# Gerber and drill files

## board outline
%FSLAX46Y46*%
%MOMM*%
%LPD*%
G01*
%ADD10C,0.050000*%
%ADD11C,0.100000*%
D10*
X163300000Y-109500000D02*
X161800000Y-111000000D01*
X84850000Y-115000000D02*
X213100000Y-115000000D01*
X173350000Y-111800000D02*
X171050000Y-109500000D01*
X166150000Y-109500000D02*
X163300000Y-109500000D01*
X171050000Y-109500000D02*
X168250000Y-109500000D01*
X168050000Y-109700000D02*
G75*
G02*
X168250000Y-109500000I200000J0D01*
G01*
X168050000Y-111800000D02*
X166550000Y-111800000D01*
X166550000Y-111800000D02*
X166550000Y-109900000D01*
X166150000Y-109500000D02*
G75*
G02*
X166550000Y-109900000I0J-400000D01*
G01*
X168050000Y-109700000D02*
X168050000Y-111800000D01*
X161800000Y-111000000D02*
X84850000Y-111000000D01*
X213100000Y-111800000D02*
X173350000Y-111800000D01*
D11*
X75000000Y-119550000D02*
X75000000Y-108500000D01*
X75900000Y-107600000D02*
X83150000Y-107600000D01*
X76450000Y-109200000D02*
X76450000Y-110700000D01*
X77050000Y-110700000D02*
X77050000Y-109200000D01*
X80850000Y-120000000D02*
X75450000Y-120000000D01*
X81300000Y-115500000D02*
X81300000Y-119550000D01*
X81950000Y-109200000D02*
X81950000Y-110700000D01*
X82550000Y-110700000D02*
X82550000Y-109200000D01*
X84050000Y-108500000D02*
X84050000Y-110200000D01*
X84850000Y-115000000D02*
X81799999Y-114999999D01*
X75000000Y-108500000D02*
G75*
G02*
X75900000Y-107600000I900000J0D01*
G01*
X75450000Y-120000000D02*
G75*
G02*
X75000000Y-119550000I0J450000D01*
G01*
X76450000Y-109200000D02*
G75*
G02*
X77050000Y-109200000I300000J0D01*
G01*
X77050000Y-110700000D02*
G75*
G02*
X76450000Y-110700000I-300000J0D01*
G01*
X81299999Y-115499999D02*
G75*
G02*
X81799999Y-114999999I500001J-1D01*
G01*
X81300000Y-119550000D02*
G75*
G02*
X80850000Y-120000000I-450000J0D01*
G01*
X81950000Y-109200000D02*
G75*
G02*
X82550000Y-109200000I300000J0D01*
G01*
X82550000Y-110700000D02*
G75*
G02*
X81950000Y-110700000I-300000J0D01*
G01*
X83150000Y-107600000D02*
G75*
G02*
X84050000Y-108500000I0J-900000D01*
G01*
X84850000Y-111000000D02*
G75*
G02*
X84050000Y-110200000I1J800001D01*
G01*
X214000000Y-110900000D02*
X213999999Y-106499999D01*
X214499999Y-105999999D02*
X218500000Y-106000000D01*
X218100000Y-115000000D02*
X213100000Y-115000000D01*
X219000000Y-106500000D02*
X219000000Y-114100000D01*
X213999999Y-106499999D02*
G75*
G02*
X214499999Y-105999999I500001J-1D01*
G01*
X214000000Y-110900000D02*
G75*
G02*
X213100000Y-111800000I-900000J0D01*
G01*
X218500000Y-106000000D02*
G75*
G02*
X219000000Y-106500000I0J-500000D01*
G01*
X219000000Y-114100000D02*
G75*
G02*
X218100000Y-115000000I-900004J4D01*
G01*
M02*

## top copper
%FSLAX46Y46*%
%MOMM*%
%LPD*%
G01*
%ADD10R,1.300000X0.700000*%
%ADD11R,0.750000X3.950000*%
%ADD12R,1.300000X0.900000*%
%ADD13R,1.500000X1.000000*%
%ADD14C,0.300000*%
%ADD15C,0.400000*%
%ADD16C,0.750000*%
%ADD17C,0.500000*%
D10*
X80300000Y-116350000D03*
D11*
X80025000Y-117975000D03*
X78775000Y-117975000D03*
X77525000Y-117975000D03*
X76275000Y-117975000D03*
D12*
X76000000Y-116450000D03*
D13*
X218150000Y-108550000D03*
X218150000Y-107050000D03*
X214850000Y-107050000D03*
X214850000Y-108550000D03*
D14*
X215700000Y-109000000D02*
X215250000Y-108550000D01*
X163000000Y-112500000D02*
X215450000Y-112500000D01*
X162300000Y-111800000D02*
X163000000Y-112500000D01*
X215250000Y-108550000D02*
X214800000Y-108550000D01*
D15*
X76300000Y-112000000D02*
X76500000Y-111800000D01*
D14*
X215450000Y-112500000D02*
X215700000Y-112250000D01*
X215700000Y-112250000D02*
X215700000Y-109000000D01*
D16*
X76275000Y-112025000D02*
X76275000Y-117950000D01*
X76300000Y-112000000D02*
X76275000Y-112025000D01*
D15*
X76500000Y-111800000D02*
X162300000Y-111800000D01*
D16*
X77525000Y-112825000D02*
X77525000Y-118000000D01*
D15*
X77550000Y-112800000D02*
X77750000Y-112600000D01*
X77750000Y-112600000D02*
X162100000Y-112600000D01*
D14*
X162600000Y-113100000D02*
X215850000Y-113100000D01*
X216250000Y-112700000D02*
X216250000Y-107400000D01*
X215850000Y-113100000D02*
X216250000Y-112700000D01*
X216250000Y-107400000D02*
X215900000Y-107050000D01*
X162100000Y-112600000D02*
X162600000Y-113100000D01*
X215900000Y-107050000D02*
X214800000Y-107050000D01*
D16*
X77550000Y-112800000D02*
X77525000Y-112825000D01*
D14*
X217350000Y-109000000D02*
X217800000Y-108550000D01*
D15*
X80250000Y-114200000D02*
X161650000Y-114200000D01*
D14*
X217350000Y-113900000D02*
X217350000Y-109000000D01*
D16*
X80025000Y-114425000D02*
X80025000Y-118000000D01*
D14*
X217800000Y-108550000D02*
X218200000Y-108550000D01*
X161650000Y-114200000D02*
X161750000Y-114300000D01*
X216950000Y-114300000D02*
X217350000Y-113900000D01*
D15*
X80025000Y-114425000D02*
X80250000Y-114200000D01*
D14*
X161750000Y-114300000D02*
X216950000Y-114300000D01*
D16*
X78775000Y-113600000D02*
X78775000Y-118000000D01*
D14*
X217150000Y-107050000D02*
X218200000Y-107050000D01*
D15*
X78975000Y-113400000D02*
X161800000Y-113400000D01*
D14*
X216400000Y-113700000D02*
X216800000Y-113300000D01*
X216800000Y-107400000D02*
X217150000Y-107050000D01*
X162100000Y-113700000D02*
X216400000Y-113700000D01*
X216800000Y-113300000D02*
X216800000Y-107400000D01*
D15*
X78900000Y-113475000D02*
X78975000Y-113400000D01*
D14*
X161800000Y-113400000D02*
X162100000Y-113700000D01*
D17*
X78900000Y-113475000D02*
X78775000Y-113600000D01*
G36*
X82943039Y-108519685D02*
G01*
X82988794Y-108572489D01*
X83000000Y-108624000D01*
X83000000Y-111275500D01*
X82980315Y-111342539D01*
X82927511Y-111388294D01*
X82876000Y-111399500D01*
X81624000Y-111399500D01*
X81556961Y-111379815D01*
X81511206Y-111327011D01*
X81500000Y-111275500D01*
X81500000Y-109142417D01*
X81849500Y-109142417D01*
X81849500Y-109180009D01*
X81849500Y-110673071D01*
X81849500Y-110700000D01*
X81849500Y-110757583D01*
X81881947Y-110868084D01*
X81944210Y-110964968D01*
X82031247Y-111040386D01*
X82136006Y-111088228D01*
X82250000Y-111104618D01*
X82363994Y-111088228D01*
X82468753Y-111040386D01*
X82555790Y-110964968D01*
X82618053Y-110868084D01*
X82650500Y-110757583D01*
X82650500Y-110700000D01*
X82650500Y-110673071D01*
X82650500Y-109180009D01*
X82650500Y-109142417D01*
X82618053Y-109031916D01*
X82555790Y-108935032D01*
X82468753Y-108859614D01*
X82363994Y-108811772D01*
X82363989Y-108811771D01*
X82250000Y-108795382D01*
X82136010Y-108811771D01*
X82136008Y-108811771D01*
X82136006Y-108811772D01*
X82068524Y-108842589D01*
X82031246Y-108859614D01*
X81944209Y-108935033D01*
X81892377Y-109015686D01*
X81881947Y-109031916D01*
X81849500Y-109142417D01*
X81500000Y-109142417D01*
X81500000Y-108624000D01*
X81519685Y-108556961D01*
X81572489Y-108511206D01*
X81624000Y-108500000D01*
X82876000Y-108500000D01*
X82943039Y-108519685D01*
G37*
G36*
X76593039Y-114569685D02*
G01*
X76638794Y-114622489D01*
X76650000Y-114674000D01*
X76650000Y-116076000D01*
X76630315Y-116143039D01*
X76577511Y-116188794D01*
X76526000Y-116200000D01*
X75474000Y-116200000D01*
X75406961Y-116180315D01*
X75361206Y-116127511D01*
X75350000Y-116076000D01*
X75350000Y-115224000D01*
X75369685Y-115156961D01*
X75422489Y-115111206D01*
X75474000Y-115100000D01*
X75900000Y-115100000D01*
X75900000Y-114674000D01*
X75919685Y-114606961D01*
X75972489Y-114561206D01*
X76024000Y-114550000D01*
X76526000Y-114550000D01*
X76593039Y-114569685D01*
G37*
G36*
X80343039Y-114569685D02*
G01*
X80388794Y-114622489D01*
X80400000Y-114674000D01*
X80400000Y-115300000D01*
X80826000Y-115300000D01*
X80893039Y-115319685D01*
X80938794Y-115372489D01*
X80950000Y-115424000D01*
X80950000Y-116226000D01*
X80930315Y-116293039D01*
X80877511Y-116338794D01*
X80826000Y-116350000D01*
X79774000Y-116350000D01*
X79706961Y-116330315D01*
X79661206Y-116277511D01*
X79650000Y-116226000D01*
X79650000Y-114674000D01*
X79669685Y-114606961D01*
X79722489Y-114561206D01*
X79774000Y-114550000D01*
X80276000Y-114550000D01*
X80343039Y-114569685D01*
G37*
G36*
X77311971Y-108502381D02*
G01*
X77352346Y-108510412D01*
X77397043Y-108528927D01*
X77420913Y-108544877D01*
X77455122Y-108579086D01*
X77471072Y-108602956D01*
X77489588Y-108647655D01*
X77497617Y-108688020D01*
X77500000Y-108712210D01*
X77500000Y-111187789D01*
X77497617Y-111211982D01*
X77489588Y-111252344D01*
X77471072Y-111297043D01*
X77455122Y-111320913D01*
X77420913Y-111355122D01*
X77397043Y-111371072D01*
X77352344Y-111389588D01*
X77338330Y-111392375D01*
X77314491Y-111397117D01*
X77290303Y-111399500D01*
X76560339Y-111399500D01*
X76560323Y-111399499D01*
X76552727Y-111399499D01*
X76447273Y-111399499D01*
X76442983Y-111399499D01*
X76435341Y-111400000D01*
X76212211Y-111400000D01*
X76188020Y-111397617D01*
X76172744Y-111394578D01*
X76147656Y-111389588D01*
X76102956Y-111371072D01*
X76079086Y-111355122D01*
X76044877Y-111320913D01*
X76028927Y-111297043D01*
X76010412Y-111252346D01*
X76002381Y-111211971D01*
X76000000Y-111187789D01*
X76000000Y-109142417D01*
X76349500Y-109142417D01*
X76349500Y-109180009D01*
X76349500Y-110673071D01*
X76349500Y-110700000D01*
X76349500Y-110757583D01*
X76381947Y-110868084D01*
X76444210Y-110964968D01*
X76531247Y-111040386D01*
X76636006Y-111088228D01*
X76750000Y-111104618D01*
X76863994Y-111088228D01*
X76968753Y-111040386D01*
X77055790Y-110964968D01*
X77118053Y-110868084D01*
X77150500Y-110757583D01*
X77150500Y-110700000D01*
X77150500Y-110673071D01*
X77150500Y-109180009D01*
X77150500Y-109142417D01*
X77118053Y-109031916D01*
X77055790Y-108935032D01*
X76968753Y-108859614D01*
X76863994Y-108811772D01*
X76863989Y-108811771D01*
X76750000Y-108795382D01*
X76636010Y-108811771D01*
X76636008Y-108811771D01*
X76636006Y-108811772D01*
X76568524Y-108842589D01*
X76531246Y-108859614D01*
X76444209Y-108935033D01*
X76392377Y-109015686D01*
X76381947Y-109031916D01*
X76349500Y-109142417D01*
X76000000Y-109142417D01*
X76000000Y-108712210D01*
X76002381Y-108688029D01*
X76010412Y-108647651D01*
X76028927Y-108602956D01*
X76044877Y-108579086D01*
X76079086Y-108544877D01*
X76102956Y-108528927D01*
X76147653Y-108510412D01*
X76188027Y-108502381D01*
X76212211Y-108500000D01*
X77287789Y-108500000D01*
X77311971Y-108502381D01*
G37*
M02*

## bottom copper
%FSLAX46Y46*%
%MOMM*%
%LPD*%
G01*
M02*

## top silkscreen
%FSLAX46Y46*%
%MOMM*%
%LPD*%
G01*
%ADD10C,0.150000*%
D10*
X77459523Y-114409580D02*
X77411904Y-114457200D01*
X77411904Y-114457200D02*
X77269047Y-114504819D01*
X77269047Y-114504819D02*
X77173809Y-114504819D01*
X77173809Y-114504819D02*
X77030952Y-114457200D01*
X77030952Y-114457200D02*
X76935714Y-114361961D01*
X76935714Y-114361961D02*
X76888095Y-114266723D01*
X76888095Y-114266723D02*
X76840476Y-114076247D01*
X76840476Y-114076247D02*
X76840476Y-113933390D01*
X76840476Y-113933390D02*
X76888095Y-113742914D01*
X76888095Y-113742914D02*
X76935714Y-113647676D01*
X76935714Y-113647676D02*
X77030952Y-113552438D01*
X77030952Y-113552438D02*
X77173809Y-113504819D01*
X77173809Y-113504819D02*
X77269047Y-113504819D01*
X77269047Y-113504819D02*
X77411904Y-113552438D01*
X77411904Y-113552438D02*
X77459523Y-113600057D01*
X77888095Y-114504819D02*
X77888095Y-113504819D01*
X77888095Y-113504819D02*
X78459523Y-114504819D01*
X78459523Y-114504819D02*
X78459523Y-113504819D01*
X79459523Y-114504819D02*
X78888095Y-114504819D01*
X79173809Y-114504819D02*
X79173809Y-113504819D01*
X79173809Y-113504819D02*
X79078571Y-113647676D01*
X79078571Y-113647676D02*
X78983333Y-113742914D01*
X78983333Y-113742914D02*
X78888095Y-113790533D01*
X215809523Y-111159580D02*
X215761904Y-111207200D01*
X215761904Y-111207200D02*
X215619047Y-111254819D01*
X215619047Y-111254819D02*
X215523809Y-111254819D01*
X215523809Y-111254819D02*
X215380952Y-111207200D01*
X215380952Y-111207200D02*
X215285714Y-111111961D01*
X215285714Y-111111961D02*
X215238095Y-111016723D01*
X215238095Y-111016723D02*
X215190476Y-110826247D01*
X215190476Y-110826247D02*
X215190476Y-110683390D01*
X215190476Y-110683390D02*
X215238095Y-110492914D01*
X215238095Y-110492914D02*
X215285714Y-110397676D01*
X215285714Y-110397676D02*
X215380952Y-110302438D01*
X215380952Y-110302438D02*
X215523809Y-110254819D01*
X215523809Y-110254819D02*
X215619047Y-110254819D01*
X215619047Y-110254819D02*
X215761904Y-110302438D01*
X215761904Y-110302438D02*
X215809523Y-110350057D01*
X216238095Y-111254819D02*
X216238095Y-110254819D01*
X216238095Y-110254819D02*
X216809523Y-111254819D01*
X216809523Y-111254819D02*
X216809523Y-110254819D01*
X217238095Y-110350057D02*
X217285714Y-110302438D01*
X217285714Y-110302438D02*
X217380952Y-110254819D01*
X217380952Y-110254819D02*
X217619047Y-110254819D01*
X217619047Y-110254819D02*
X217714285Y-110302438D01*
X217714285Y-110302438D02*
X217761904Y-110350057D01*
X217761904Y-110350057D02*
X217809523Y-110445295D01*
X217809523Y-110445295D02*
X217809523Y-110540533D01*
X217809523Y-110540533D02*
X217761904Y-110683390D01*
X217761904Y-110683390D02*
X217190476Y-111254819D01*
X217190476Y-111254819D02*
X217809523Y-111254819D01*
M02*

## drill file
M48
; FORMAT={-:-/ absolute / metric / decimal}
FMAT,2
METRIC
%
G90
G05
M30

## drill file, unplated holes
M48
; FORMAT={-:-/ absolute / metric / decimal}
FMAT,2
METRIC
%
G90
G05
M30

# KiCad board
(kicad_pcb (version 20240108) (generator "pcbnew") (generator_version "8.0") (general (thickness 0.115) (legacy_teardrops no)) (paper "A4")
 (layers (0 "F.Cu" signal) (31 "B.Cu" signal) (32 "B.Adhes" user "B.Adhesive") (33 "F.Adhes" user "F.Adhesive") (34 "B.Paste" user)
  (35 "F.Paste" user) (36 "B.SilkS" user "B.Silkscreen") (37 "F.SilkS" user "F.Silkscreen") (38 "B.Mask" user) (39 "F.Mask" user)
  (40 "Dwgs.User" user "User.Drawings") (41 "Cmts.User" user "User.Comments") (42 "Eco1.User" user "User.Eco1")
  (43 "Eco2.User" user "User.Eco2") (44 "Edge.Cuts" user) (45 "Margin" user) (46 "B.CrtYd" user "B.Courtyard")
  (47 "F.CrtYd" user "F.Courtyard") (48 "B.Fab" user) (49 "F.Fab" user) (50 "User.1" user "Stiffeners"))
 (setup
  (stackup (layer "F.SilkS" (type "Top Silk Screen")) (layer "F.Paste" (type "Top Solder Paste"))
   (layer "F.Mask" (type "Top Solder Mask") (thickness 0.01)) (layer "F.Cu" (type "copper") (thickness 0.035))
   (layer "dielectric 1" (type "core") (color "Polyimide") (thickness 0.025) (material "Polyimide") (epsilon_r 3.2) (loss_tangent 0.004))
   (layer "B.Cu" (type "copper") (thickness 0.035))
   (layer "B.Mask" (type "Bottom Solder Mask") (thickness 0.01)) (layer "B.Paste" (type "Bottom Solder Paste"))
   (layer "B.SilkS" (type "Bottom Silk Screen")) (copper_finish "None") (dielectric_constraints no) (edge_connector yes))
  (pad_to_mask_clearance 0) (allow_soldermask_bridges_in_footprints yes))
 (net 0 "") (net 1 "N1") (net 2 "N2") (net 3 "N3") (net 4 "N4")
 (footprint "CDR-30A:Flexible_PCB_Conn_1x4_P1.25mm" (layer "F.Cu") (at 78.15 116 180)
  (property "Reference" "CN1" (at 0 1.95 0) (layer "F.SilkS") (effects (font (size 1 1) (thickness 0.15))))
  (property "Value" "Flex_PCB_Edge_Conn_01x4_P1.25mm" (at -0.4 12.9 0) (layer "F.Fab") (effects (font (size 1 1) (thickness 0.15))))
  (fp_line (start 3.15 -3.55) (end 3.15 7.5) (stroke (width 0.1) (type default)) (layer "Edge.Cuts"))
  (fp_line (start 2.25 8.4) (end -5 8.4) (stroke (width 0.1) (type default)) (layer "Edge.Cuts"))
  (fp_line (start 1.7 6.8) (end 1.7 5.3) (stroke (width 0.1) (type default)) (layer "Edge.Cuts"))
  (fp_line (start 1.1 5.3) (end 1.1 6.8) (stroke (width 0.1) (type default)) (layer "Edge.Cuts"))
  (fp_line (start -2.7 -4) (end 2.7 -4) (stroke (width 0.1) (type default)) (layer "Edge.Cuts"))
  (fp_line (start -3.15 0.5) (end -3.15 -3.55) (stroke (width 0.1) (type default)) (layer "Edge.Cuts"))
  (fp_line (start -3.8 6.8) (end -3.8 5.3) (stroke (width 0.1) (type default)) (layer "Edge.Cuts"))
  (fp_line (start -4.4 5.3) (end -4.4 6.8) (stroke (width 0.1) (type default)) (layer "Edge.Cuts"))
  (fp_line (start -5.9 7.5) (end -5.9 5.8) (stroke (width 0.1) (type default)) (layer "Edge.Cuts"))
  (fp_line (start -6.7 1) (end -3.649999 1.000001) (stroke (width 0.1) (type default)) (layer "Edge.Cuts"))
  (fp_arc (start 3.15 7.5) (mid 2.886396 8.136396) (end 2.25 8.4) (stroke (width 0.1) (type default)) (layer "Edge.Cuts"))
  (fp_arc (start 2.7 -4) (mid 3.018198 -3.868198) (end 3.15 -3.55) (stroke (width 0.1) (type default)) (layer "Edge.Cuts"))
  (fp_arc (start 1.7 6.8) (mid 1.4 7.1) (end 1.1 6.8) (stroke (width 0.1) (type default)) (layer "Edge.Cuts"))
  (fp_arc (start 1.1 5.3) (mid 1.4 5) (end 1.7 5.3) (stroke (width 0.1) (type default)) (layer "Edge.Cuts"))
  (fp_arc (start -3.149999 0.500001) (mid -3.296446 0.853554) (end -3.649999 1.000001) (stroke (width 0.1) (type default))
   (layer "Edge.Cuts"))
  (fp_arc (start -3.15 -3.55) (mid -3.018198 -3.868198) (end -2.7 -4) (stroke (width 0.1) (type default)) (layer "Edge.Cuts"))
  (fp_arc (start -3.8 6.8) (mid -4.1 7.1) (end -4.4 6.8) (stroke (width 0.1) (type default)) (layer "Edge.Cuts"))
  (fp_arc (start -4.4 5.3) (mid -4.1 5) (end -3.8 5.3) (stroke (width 0.1) (type default)) (layer "Edge.Cuts"))
  (fp_arc (start -5 8.4) (mid -5.636396 8.136396) (end -5.9 7.5) (stroke (width 0.1) (type default)) (layer "Edge.Cuts"))
  (fp_arc (start -6.7 5) (mid -6.134315 5.234315) (end -5.9 5.8) (stroke (width 0.1) (type default)) (layer "Edge.Cuts"))
  (pad "1" connect rect (at -2.15 -0.35 180) (size 1.3 0.7) (layers "F.Cu" "F.Mask") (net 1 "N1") (thermal_bridge_angle 45))
  (pad "1" connect rect (at -1.875 -1.975 180) (size 0.75 3.95) (layers "F.Cu" "F.Mask") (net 1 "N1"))
  (pad "2" connect rect (at -0.625 -1.975 180) (size 0.75 3.95) (layers "F.Cu" "F.Mask") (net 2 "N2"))
  (pad "3" connect rect (at 0.625 -1.975 180) (size 0.75 3.95) (layers "F.Cu" "F.Mask") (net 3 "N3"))
  (pad "4" connect rect (at 1.875 -1.975 180) (size 0.75 3.95) (layers "F.Cu" "F.Mask") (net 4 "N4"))
  (pad "4" connect rect (at 2.15 -0.45 180) (size 1.3 0.9) (layers "F.Cu" "F.Mask") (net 4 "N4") (thermal_bridge_angle 45)))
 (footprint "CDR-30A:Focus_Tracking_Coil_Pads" (layer "F.Cu") (at 216.5 107.8)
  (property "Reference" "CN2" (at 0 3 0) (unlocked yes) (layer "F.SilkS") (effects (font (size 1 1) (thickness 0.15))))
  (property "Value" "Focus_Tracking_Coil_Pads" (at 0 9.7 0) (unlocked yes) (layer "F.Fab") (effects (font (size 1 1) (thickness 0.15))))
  (fp_line (start -2.5 3.1) (end -2.500001 -1.300001) (stroke (width 0.1) (type default)) (layer "Edge.Cuts"))
  (fp_line (start -2.000001 -1.800001) (end 2 -1.8) (stroke (width 0.1) (type default)) (layer "Edge.Cuts"))
  (fp_line (start 1.6 7.2) (end -3.4 7.2) (stroke (width 0.1) (type default)) (layer "Edge.Cuts"))
  (fp_line (start 2.5 -1.3) (end 2.5 6.3) (stroke (width 0.1) (type default)) (layer "Edge.Cuts"))
  (fp_arc (start -2.500001 -1.300001) (mid -2.353554 -1.653554) (end -2.000001 -1.800001) (stroke (width 0.1) (type default))
   (layer "Edge.Cuts"))
  (fp_arc (start -2.5 3.1) (mid -2.763604 3.736396) (end -3.4 4) (stroke (width 0.1) (type default)) (layer "Edge.Cuts"))
  (fp_arc (start 2 -1.8) (mid 2.353553 -1.653553) (end 2.5 -1.3) (stroke (width 0.1) (type default)) (layer "Edge.Cuts"))
  (fp_arc (start 2.5 6.3) (mid 2.236395 6.936395) (end 1.6 7.2) (stroke (width 0.1) (type default)) (layer "Edge.Cuts"))
  (pad "1" smd rect (at 1.65 0.75) (size 1.5 1) (layers "F.Cu" "F.Paste" "F.Mask") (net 1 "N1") (thermal_bridge_angle 45))
  (pad "2" smd rect (at 1.65 -0.75) (size 1.5 1) (layers "F.Cu" "F.Paste" "F.Mask") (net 2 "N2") (thermal_bridge_angle 45))
  (pad "3" smd rect (at -1.65 -0.75) (size 1.5 1) (layers "F.Cu" "F.Paste" "F.Mask") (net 3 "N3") (thermal_bridge_angle 45))
  (pad "4" smd rect (at -1.65 0.75) (size 1.5 1) (layers "F.Cu" "F.Paste" "F.Mask") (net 4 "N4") (thermal_bridge_angle 45)))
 (gr_line (start 163.3 109.5) (end 161.8 111) (stroke (width 0.05) (type default)) (layer "Edge.Cuts"))
 (gr_line (start 84.85 115) (end 213.1 115) (stroke (width 0.05) (type default)) (layer "Edge.Cuts"))
 (gr_line (start 173.35 111.8) (end 171.05 109.5) (stroke (width 0.05) (type default)) (layer "Edge.Cuts"))
 (gr_line (start 166.15 109.5) (end 163.3 109.5) (stroke (width 0.05) (type default)) (layer "Edge.Cuts"))
 (gr_line (start 171.05 109.5) (end 168.25 109.5) (stroke (width 0.05) (type default)) (layer "Edge.Cuts"))
 (gr_arc (start 168.05 109.7) (mid 168.108579 109.558579) (end 168.25 109.5) (stroke (width 0.05) (type default)) (layer "Edge.Cuts"))
 (gr_line (start 168.05 111.8) (end 166.55 111.8) (stroke (width 0.05) (type default)) (layer "Edge.Cuts"))
 (gr_line (start 166.55 111.8) (end 166.55 109.9) (stroke (width 0.05) (type default)) (layer "Edge.Cuts"))
 (gr_arc (start 166.15 109.5) (mid 166.432843 109.617157) (end 166.55 109.9) (stroke (width 0.05) (type default)) (layer "Edge.Cuts"))
 (gr_line (start 168.05 109.7) (end 168.05 111.8) (stroke (width 0.05) (type default)) (layer "Edge.Cuts"))
 (gr_line (start 161.8 111) (end 84.85 111) (stroke (width 0.05) (type default)) (layer "Edge.Cuts"))
 (gr_line (start 213.1 111.8) (end 173.35 111.8) (stroke (width 0.05) (type default)) (layer "Edge.Cuts"))
 (segment (start 215.7 109) (end 215.25 108.55) (width 0.3) (layer "F.Cu") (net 4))
 (segment (start 163 112.5) (end 215.45 112.5) (width 0.3) (layer "F.Cu") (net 4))
 (segment (start 162.3 111.8) (end 163 112.5) (width 0.3) (layer "F.Cu") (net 4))
 (segment (start 215.25 108.55) (end 214.8 108.55) (width 0.3) (layer "F.Cu") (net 4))
 (segment (start 76.3 112) (end 76.5 111.8) (width 0.4) (layer "F.Cu") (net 4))
 (segment (start 215.45 112.5) (end 215.7 112.25) (width 0.3) (layer "F.Cu") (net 4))
 (segment (start 215.7 112.25) (end 215.7 109) (width 0.3) (layer "F.Cu") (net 4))
 (segment (start 76.275 112.025) (end 76.275 117.95) (width 0.75) (layer "F.Cu") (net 4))
 (segment (start 76.3 112) (end 76.275 112.025) (width 0.75) (layer "F.Cu") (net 4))
 (segment (start 76.5 111.8) (end 162.3 111.8) (width 0.4) (layer "F.Cu") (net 4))
 (segment (start 77.525 112.825) (end 77.525 118) (width 0.75) (layer "F.Cu") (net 3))
 (segment (start 77.55 112.8) (end 77.75 112.6) (width 0.4) (layer "F.Cu") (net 3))
 (segment (start 77.75 112.6) (end 162.1 112.6) (width 0.4) (layer "F.Cu") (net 3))
 (segment (start 162.6 113.1) (end 215.85 113.1) (width 0.3) (layer "F.Cu") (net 3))
 (segment (start 216.25 112.7) (end 216.25 107.4) (width 0.3) (layer "F.Cu") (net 3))
 (segment (start 215.85 113.1) (end 216.25 112.7) (width 0.3) (layer "F.Cu") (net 3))
 (segment (start 216.25 107.4) (end 215.9 107.05) (width 0.3) (layer "F.Cu") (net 3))
 (segment (start 162.1 112.6) (end 162.6 113.1) (width 0.3) (layer "F.Cu") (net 3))
 (segment (start 215.9 107.05) (end 214.8 107.05) (width 0.3) (layer "F.Cu") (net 3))
 (segment (start 77.55 112.8) (end 77.525 112.825) (width 0.75) (layer "F.Cu") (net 3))
 (segment (start 217.35 109) (end 217.8 108.55) (width 0.3) (layer "F.Cu") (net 1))
 (segment (start 80.25 114.2) (end 161.65 114.2) (width 0.4) (layer "F.Cu") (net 1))
 (segment (start 217.35 113.9) (end 217.35 109) (width 0.3) (layer "F.Cu") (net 1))
 (segment (start 80.025 114.425) (end 80.025 118) (width 0.75) (layer "F.Cu") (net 1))
 (segment (start 217.8 108.55) (end 218.2 108.55) (width 0.3) (layer "F.Cu") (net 1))
 (segment (start 161.65 114.2) (end 161.75 114.3) (width 0.3) (layer "F.Cu") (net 1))
 (segment (start 216.95 114.3) (end 217.35 113.9) (width 0.3) (layer "F.Cu") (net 1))
 (segment (start 80.025 114.425) (end 80.25 114.2) (width 0.4) (layer "F.Cu") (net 1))
 (segment (start 161.75 114.3) (end 216.95 114.3) (width 0.3) (layer "F.Cu") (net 1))
 (segment (start 78.775 113.6) (end 78.775 118) (width 0.75) (layer "F.Cu") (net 2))
 (segment (start 217.15 107.05) (end 218.2 107.05) (width 0.3) (layer "F.Cu") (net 2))
 (segment (start 78.975 113.4) (end 161.8 113.4) (width 0.4) (layer "F.Cu") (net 2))
 (segment (start 216.4 113.7) (end 216.8 113.3) (width 0.3) (layer "F.Cu") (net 2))
 (segment (start 216.8 107.4) (end 217.15 107.05) (width 0.3) (layer "F.Cu") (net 2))
 (segment (start 162.1 113.7) (end 216.4 113.7) (width 0.3) (layer "F.Cu") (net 2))
 (segment (start 216.8 113.3) (end 216.8 107.4) (width 0.3) (layer "F.Cu") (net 2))
 (segment (start 78.9 113.475) (end 78.975 113.4) (width 0.4) (layer "F.Cu") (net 2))
 (segment (start 161.8 113.4) (end 162.1 113.7) (width 0.3) (layer "F.Cu") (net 2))
 (segment (start 78.9 113.475) (end 78.775 113.6) (width 0.5) (layer "F.Cu") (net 2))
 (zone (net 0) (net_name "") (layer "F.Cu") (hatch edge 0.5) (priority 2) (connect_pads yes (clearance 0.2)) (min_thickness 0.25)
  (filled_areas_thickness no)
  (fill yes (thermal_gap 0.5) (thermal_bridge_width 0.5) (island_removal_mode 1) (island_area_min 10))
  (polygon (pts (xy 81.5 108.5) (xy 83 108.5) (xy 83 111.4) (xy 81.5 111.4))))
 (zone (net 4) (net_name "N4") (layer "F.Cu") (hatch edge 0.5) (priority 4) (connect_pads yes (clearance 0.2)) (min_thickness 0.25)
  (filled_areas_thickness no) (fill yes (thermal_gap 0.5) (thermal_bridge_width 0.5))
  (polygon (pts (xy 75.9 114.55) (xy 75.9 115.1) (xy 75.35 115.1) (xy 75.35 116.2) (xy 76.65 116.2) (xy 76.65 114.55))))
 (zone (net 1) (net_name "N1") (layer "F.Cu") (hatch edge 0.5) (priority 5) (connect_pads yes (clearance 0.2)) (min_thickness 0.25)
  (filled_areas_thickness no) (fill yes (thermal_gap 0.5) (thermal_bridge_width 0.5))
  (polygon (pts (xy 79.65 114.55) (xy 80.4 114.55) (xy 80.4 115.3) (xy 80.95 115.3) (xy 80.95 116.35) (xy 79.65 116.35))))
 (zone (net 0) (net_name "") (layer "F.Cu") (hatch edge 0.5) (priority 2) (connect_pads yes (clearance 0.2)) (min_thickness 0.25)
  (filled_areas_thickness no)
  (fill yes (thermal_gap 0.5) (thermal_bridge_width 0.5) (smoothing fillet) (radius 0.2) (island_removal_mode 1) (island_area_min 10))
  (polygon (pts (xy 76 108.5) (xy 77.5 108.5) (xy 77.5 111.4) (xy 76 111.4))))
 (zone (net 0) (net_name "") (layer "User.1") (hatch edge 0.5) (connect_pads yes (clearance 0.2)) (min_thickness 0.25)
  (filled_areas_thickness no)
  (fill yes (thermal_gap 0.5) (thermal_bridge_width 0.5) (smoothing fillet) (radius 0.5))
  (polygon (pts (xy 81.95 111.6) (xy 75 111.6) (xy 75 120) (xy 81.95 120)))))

